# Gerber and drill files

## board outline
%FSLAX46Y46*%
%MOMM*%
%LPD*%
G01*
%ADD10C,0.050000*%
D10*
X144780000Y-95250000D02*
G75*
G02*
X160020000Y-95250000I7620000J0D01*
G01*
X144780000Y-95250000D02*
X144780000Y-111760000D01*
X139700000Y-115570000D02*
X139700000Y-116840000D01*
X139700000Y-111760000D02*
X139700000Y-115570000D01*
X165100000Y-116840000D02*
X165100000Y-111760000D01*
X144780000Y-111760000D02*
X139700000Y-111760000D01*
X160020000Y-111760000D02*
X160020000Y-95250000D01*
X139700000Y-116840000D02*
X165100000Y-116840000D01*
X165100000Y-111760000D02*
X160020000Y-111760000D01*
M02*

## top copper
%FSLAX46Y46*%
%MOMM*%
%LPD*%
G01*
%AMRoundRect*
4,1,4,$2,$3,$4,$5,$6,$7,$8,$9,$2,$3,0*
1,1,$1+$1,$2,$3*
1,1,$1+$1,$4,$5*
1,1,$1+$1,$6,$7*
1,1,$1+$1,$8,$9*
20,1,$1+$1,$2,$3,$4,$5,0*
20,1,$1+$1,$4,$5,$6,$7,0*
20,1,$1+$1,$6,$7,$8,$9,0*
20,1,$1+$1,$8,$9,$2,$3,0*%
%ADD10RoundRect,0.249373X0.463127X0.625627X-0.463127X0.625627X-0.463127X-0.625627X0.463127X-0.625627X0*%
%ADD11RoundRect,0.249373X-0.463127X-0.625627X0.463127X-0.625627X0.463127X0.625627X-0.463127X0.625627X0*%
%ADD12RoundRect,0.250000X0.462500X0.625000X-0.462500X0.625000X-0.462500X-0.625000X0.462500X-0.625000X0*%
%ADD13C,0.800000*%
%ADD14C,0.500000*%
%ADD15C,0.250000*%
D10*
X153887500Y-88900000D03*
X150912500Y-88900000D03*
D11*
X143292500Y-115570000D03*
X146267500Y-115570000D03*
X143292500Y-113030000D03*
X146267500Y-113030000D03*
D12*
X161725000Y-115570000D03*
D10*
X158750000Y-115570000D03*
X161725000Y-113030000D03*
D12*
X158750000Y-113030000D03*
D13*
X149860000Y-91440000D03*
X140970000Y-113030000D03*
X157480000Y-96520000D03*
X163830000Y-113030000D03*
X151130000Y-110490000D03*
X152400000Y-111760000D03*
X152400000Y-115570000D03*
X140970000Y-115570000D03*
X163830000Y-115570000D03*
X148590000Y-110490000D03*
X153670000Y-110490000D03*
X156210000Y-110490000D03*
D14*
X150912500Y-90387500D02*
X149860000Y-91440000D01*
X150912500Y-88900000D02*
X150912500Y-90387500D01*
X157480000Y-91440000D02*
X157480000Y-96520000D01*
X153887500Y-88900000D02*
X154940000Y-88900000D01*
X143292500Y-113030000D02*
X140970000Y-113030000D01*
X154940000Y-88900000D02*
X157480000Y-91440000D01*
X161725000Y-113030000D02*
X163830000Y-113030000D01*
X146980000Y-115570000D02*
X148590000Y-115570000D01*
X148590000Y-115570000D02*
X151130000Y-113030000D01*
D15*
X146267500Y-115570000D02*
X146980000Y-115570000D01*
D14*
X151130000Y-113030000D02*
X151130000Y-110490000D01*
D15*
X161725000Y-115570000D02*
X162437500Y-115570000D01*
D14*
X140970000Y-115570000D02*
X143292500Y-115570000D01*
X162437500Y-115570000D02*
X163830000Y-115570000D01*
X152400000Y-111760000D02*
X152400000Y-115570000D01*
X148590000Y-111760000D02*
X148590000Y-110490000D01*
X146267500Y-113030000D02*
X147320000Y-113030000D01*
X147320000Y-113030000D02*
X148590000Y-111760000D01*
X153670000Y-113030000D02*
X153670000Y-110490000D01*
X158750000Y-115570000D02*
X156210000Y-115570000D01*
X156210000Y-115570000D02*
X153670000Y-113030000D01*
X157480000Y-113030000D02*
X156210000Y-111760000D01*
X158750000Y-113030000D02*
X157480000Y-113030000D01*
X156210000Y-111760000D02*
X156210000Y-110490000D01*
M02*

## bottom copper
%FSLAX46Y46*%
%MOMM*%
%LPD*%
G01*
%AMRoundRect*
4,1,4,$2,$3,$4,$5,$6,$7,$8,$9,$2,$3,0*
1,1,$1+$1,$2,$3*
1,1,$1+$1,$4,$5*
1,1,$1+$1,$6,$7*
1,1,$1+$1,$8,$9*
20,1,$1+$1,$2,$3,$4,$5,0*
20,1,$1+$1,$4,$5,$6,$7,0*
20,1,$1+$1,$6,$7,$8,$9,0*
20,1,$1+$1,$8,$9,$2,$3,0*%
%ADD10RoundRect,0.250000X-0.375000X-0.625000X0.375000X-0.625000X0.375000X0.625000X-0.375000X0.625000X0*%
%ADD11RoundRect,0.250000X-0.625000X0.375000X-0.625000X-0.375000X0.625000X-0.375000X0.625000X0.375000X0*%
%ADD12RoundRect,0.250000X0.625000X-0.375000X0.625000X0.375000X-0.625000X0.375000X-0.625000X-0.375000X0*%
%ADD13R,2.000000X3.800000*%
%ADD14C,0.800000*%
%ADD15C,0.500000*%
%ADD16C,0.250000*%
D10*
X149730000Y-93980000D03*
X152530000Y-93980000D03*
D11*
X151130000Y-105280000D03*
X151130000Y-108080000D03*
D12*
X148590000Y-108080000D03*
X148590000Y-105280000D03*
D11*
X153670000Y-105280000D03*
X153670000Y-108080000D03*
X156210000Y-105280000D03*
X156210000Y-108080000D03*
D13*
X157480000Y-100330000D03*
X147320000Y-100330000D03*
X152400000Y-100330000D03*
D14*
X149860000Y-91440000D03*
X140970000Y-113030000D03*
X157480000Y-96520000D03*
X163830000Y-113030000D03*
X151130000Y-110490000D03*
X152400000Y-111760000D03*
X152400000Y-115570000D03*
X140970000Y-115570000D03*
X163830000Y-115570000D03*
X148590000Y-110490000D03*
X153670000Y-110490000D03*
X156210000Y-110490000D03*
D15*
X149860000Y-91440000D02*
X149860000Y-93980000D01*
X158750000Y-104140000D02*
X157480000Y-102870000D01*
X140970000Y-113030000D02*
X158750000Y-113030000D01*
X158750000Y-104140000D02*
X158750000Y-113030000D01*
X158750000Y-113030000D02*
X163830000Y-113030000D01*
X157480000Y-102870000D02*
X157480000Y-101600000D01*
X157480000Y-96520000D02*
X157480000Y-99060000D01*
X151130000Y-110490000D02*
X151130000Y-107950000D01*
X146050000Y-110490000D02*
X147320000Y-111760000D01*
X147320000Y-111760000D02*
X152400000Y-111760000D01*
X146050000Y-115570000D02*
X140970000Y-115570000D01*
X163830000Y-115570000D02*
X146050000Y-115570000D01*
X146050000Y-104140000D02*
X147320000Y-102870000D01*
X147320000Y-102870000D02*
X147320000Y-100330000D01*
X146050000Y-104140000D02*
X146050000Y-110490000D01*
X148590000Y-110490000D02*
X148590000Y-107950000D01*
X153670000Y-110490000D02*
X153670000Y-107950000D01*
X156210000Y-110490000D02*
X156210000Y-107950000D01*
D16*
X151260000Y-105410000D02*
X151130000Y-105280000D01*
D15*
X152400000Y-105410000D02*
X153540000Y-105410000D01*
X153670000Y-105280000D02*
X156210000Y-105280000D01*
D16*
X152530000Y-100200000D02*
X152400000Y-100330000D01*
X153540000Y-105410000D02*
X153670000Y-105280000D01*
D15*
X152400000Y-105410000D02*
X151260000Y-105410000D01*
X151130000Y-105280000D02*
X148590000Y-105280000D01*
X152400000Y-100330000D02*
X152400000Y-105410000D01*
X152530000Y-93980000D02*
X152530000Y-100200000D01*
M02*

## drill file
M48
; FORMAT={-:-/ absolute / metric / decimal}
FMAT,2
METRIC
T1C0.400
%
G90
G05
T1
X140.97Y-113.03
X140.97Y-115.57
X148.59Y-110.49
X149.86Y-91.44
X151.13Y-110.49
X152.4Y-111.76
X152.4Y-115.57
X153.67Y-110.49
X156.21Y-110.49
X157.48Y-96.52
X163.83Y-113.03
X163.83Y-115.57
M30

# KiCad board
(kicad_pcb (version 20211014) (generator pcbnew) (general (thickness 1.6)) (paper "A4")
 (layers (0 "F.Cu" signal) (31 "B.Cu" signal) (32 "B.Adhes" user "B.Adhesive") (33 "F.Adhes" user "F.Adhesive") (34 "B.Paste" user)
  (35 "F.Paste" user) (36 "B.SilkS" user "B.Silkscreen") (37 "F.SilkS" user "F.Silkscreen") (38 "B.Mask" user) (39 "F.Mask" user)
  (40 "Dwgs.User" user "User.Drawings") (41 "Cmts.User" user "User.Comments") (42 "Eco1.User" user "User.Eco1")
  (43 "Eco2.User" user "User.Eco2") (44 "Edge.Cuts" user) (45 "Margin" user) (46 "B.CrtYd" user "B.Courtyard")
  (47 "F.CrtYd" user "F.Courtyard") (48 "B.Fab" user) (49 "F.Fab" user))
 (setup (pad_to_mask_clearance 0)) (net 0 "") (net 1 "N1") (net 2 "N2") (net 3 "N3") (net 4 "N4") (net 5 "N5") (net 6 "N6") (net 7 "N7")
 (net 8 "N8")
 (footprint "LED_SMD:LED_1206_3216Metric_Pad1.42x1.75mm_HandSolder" (layer "F.Cu") (at 152.4 88.9 180)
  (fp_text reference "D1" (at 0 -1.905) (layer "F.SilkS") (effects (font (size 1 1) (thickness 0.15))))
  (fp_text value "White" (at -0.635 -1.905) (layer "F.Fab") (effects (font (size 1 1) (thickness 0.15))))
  (pad "1" smd roundrect locked (at -1.4875 0 180) (size 1.425 1.75) (layers "F.Cu" "F.Paste" "F.Mask") (roundrect_rratio 0.1749985965)
   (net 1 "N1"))
  (pad "2" smd roundrect locked (at 1.4875 0 180) (size 1.425 1.75) (layers "F.Cu" "F.Paste" "F.Mask") (roundrect_rratio 0.1749985965)
   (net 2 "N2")))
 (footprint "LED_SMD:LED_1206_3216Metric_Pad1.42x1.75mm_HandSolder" (layer "F.Cu") (at 144.78 115.57)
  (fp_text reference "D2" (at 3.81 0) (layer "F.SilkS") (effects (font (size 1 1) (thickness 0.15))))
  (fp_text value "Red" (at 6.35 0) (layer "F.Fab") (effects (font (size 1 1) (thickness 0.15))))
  (pad "1" smd roundrect locked (at -1.4875 0) (size 1.425 1.75) (layers "F.Cu" "F.Paste" "F.Mask") (roundrect_rratio 0.1749985965)
   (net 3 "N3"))
  (pad "2" smd roundrect locked (at 1.4875 0) (size 1.425 1.75) (layers "F.Cu" "F.Paste" "F.Mask") (roundrect_rratio 0.1749985965)
   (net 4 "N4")))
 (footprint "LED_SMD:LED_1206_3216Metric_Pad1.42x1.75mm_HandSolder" (layer "F.Cu") (at 144.78 113.03)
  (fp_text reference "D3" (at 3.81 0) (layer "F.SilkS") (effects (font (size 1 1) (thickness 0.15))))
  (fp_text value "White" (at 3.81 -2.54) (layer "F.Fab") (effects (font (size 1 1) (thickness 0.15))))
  (pad "1" smd roundrect locked (at -1.4875 0) (size 1.425 1.75) (layers "F.Cu" "F.Paste" "F.Mask") (roundrect_rratio 0.1749985965)
   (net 1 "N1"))
  (pad "2" smd roundrect locked (at 1.4875 0) (size 1.425 1.75) (layers "F.Cu" "F.Paste" "F.Mask") (roundrect_rratio 0.1749985965)
   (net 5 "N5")))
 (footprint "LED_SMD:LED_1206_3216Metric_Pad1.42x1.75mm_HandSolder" (layer "F.Cu") (at 160.2375 115.57 180)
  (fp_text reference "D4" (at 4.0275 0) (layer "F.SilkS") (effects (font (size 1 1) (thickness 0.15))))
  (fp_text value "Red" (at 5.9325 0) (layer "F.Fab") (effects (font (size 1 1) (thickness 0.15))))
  (pad "1" smd roundrect locked (at -1.4875 0 180) (size 1.425 1.75) (layers "F.Cu" "F.Paste" "F.Mask") (roundrect_rratio 0.1754385965)
   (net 3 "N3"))
  (pad "2" smd roundrect locked (at 1.4875 0 180) (size 1.425 1.75) (layers "F.Cu" "F.Paste" "F.Mask") (roundrect_rratio 0.1749985965)
   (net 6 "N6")))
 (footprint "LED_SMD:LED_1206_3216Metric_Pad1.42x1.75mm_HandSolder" (layer "F.Cu") (at 160.2375 113.03 180)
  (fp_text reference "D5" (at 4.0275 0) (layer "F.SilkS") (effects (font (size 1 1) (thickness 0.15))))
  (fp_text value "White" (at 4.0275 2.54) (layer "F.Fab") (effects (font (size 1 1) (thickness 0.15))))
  (pad "1" smd roundrect locked (at -1.4875 0 180) (size 1.425 1.75) (layers "F.Cu" "F.Paste" "F.Mask") (roundrect_rratio 0.1749985965)
   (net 1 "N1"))
  (pad "2" smd roundrect locked (at 1.4875 0 180) (size 1.425 1.75) (layers "F.Cu" "F.Paste" "F.Mask") (roundrect_rratio 0.1754385965)
   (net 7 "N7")))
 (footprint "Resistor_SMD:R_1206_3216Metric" (layer "B.Cu") (at 151.13 93.98)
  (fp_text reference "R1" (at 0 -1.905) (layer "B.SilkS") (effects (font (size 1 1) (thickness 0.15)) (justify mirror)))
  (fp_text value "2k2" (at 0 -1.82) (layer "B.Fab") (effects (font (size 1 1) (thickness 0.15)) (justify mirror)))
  (pad "1" smd roundrect locked (at -1.4 0) (size 1.25 1.75) (layers "B.Cu" "B.Paste" "B.Mask") (roundrect_rratio 0.2) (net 2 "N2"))
  (pad "2" smd roundrect locked (at 1.4 0) (size 1.25 1.75) (layers "B.Cu" "B.Paste" "B.Mask") (roundrect_rratio 0.2) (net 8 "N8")))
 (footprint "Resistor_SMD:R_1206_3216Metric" (layer "B.Cu") (at 151.13 106.68 -90)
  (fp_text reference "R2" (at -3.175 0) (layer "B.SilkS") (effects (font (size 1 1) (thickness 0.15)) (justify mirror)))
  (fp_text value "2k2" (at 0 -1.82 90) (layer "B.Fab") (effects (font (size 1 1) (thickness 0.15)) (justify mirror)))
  (pad "1" smd roundrect locked (at -1.4 0 270) (size 1.25 1.75) (layers "B.Cu" "B.Paste" "B.Mask") (roundrect_rratio 0.2) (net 8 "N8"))
  (pad "2" smd roundrect locked (at 1.4 0 270) (size 1.25 1.75) (layers "B.Cu" "B.Paste" "B.Mask") (roundrect_rratio 0.2) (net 4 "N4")))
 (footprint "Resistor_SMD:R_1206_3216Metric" (layer "B.Cu") (at 148.59 106.68 90)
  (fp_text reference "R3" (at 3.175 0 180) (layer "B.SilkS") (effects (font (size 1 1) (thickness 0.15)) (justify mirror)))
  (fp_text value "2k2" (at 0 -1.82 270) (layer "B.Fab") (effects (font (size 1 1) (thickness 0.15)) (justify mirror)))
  (pad "1" smd roundrect locked (at -1.4 0 90) (size 1.25 1.75) (layers "B.Cu" "B.Paste" "B.Mask") (roundrect_rratio 0.2) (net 5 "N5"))
  (pad "2" smd roundrect locked (at 1.4 0 90) (size 1.25 1.75) (layers "B.Cu" "B.Paste" "B.Mask") (roundrect_rratio 0.2) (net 8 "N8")))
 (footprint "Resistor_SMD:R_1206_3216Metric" (layer "B.Cu") (at 153.67 106.68 -90)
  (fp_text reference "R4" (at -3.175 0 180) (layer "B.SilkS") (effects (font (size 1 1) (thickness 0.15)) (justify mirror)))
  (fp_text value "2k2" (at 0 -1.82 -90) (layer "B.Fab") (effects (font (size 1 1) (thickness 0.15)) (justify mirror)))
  (pad "1" smd roundrect locked (at -1.4 0 270) (size 1.25 1.75) (layers "B.Cu" "B.Paste" "B.Mask") (roundrect_rratio 0.2) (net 8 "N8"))
  (pad "2" smd roundrect locked (at 1.4 0 270) (size 1.25 1.75) (layers "B.Cu" "B.Paste" "B.Mask") (roundrect_rratio 0.2) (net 6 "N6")))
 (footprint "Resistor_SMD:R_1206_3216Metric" (layer "B.Cu") (at 156.21 106.68 -90)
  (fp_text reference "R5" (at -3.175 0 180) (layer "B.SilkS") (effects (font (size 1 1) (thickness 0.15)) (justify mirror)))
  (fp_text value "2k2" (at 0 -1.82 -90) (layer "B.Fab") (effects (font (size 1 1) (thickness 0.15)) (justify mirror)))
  (pad "1" smd roundrect locked (at -1.4 0 270) (size 1.25 1.75) (layers "B.Cu" "B.Paste" "B.Mask") (roundrect_rratio 0.2) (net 8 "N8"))
  (pad "2" smd roundrect locked (at 1.4 0 270) (size 1.25 1.75) (layers "B.Cu" "B.Paste" "B.Mask") (roundrect_rratio 0.2) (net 7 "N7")))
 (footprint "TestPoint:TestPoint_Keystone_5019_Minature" (layer "B.Cu") (at 157.48 100.33 90)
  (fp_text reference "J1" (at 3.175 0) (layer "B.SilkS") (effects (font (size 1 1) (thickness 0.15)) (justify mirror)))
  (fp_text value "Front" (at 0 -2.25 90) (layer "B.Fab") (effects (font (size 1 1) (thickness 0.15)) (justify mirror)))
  (pad "1" smd rect locked (at 0 0 90) (size 3.8 2) (layers "B.Cu" "B.Paste" "B.Mask") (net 1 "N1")))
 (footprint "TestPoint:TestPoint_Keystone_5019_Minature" (layer "B.Cu") (at 147.32 100.33 90)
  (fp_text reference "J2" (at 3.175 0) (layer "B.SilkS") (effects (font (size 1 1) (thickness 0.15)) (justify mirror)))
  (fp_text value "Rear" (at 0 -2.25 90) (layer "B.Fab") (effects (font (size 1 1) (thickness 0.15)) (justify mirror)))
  (pad "1" smd rect locked (at 0 0 90) (size 3.8 2) (layers "B.Cu" "B.Paste" "B.Mask") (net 3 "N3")))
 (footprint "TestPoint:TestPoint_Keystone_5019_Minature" (layer "B.Cu") (at 152.4 100.33 90)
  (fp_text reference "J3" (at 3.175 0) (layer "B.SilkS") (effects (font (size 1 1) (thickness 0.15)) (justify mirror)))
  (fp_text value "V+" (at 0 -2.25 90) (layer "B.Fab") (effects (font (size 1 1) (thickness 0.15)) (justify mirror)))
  (pad "1" smd rect locked (at 0 0 90) (size 3.8 2) (layers "B.Cu" "B.Paste" "B.Mask") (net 8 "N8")))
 (gr_arc (start 144.78 95.25) (mid 152.4 87.63) (end 160.02 95.25) (layer "Edge.Cuts") (width 0.05))
 (gr_line (start 144.78 95.25) (end 144.78 111.76) (layer "Edge.Cuts") (width 0.05))
 (gr_line (start 139.7 115.57) (end 139.7 116.84) (layer "Edge.Cuts") (width 0.05))
 (gr_line (start 139.7 111.76) (end 139.7 115.57) (layer "Edge.Cuts") (width 0.05))
 (gr_line (start 165.1 116.84) (end 165.1 111.76) (layer "Edge.Cuts") (width 0.05))
 (gr_line (start 144.78 111.76) (end 139.7 111.76) (layer "Edge.Cuts") (width 0.05))
 (gr_line (start 160.02 111.76) (end 160.02 95.25) (layer "Edge.Cuts") (width 0.05))
 (gr_line (start 139.7 116.84) (end 165.1 116.84) (layer "Edge.Cuts") (width 0.05))
 (gr_line (start 165.1 111.76) (end 160.02 111.76) (layer "Edge.Cuts") (width 0.05))
 (segment (start 150.9125 90.3875) (end 149.86 91.44) (width 0.5) (layer "F.Cu") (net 2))
 (segment (start 150.9125 88.9) (end 150.9125 90.3875) (width 0.5) (layer "F.Cu") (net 2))
 (via (at 149.86 91.44) (size 0.8) (drill 0.4) (layers "F.Cu" "B.Cu") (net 2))
 (segment (start 149.86 91.44) (end 149.86 93.98) (width 0.5) (layer "B.Cu") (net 2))
 (segment (start 157.48 91.44) (end 157.48 96.52) (width 0.5) (layer "F.Cu") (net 1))
 (segment (start 153.8875 88.9) (end 154.94 88.9) (width 0.5) (layer "F.Cu") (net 1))
 (segment (start 143.2925 113.03) (end 140.97 113.03) (width 0.5) (layer "F.Cu") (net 1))
 (segment (start 154.94 88.9) (end 157.48 91.44) (width 0.5) (layer "F.Cu") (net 1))
 (segment (start 161.725 113.03) (end 163.83 113.03) (width 0.5) (layer "F.Cu") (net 1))
 (via (at 140.97 113.03) (size 0.8) (drill 0.4) (layers "F.Cu" "B.Cu") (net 1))
 (via (at 157.48 96.52) (size 0.8) (drill 0.4) (layers "F.Cu" "B.Cu") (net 1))
 (via (at 163.83 113.03) (size 0.8) (drill 0.4) (layers "F.Cu" "B.Cu") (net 1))
 (segment (start 158.75 104.14) (end 157.48 102.87) (width 0.5) (layer "B.Cu") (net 1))
 (segment (start 140.97 113.03) (end 158.75 113.03) (width 0.5) (layer "B.Cu") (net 1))
 (segment (start 158.75 104.14) (end 158.75 113.03) (width 0.5) (layer "B.Cu") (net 1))
 (segment (start 158.75 113.03) (end 163.83 113.03) (width 0.5) (layer "B.Cu") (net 1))
 (segment (start 157.48 102.87) (end 157.48 101.6) (width 0.5) (layer "B.Cu") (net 1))
 (segment (start 157.48 96.52) (end 157.48 99.06) (width 0.5) (layer "B.Cu") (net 1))
 (segment (start 146.98 115.57) (end 148.59 115.57) (width 0.5) (layer "F.Cu") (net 4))
 (segment (start 148.59 115.57) (end 151.13 113.03) (width 0.5) (layer "F.Cu") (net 4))
 (segment (start 146.2675 115.57) (end 146.98 115.57) (width 0.25) (layer "F.Cu") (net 4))
 (segment (start 151.13 113.03) (end 151.13 110.49) (width 0.5) (layer "F.Cu") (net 4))
 (via (at 151.13 110.49) (size 0.8) (drill 0.4) (layers "F.Cu" "B.Cu") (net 4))
 (segment (start 151.13 110.49) (end 151.13 107.95) (width 0.5) (layer "B.Cu") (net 4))
 (segment (start 161.725 115.57) (end 162.4375 115.57) (width 0.25) (layer "F.Cu") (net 3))
 (segment (start 140.97 115.57) (end 143.2925 115.57) (width 0.5) (layer "F.Cu") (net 3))
 (segment (start 162.4375 115.57) (end 163.83 115.57) (width 0.5) (layer "F.Cu") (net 3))
 (segment (start 152.4 111.76) (end 152.4 115.57) (width 0.5) (layer "F.Cu") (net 3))
 (via (at 152.4 111.76) (size 0.8) (drill 0.4) (layers "F.Cu" "B.Cu") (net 3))
 (via (at 152.4 115.57) (size 0.8) (drill 0.4) (layers "F.Cu" "B.Cu") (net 3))
 (via (at 140.97 115.57) (size 0.8) (drill 0.4) (layers "F.Cu" "B.Cu") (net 3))
 (via (at 163.83 115.57) (size 0.8) (drill 0.4) (layers "F.Cu" "B.Cu") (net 3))
 (segment (start 146.05 110.49) (end 147.32 111.76) (width 0.5) (layer "B.Cu") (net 3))
 (segment (start 147.32 111.76) (end 152.4 111.76) (width 0.5) (layer "B.Cu") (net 3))
 (segment (start 146.05 115.57) (end 140.97 115.57) (width 0.5) (layer "B.Cu") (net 3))
 (segment (start 163.83 115.57) (end 146.05 115.57) (width 0.5) (layer "B.Cu") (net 3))
 (segment (start 146.05 104.14) (end 147.32 102.87) (width 0.5) (layer "B.Cu") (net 3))
 (segment (start 147.32 102.87) (end 147.32 100.33) (width 0.5) (layer "B.Cu") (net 3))
 (segment (start 146.05 104.14) (end 146.05 110.49) (width 0.5) (layer "B.Cu") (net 3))
 (segment (start 148.59 111.76) (end 148.59 110.49) (width 0.5) (layer "F.Cu") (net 5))
 (segment (start 146.2675 113.03) (end 147.32 113.03) (width 0.5) (layer "F.Cu") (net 5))
 (segment (start 147.32 113.03) (end 148.59 111.76) (width 0.5) (layer "F.Cu") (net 5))
 (via (at 148.59 110.49) (size 0.8) (drill 0.4) (layers "F.Cu" "B.Cu") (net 5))
 (segment (start 148.59 110.49) (end 148.59 107.95) (width 0.5) (layer "B.Cu") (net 5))
 (segment (start 153.67 113.03) (end 153.67 110.49) (width 0.5) (layer "F.Cu") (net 6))
 (segment (start 158.75 115.57) (end 156.21 115.57) (width 0.5) (layer "F.Cu") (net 6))
 (segment (start 156.21 115.57) (end 153.67 113.03) (width 0.5) (layer "F.Cu") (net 6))
 (via (at 153.67 110.49) (size 0.8) (drill 0.4) (layers "F.Cu" "B.Cu") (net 6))
 (segment (start 153.67 110.49) (end 153.67 107.95) (width 0.5) (layer "B.Cu") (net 6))
 (segment (start 157.48 113.03) (end 156.21 111.76) (width 0.5) (layer "F.Cu") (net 7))
 (segment (start 158.75 113.03) (end 157.48 113.03) (width 0.5) (layer "F.Cu") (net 7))
 (segment (start 156.21 111.76) (end 156.21 110.49) (width 0.5) (layer "F.Cu") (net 7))
 (via (at 156.21 110.49) (size 0.8) (drill 0.4) (layers "F.Cu" "B.Cu") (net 7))
 (segment (start 156.21 110.49) (end 156.21 107.95) (width 0.5) (layer "B.Cu") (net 7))
 (segment (start 151.26 105.41) (end 151.13 105.28) (width 0.25) (layer "B.Cu") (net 8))
 (segment (start 152.4 105.41) (end 153.54 105.41) (width 0.5) (layer "B.Cu") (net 8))
 (segment (start 153.67 105.28) (end 156.21 105.28) (width 0.5) (layer "B.Cu") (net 8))
 (segment (start 152.53 100.2) (end 152.4 100.33) (width 0.25) (layer "B.Cu") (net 8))
 (segment (start 153.54 105.41) (end 153.67 105.28) (width 0.25) (layer "B.Cu") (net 8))
 (segment (start 152.4 105.41) (end 151.26 105.41) (width 0.5) (layer "B.Cu") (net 8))
 (segment (start 151.13 105.28) (end 148.59 105.28) (width 0.5) (layer "B.Cu") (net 8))
 (segment (start 152.4 100.33) (end 152.4 105.41) (width 0.5) (layer "B.Cu") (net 8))
 (segment (start 152.53 93.98) (end 152.53 100.2) (width 0.5) (layer "B.Cu") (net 8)))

